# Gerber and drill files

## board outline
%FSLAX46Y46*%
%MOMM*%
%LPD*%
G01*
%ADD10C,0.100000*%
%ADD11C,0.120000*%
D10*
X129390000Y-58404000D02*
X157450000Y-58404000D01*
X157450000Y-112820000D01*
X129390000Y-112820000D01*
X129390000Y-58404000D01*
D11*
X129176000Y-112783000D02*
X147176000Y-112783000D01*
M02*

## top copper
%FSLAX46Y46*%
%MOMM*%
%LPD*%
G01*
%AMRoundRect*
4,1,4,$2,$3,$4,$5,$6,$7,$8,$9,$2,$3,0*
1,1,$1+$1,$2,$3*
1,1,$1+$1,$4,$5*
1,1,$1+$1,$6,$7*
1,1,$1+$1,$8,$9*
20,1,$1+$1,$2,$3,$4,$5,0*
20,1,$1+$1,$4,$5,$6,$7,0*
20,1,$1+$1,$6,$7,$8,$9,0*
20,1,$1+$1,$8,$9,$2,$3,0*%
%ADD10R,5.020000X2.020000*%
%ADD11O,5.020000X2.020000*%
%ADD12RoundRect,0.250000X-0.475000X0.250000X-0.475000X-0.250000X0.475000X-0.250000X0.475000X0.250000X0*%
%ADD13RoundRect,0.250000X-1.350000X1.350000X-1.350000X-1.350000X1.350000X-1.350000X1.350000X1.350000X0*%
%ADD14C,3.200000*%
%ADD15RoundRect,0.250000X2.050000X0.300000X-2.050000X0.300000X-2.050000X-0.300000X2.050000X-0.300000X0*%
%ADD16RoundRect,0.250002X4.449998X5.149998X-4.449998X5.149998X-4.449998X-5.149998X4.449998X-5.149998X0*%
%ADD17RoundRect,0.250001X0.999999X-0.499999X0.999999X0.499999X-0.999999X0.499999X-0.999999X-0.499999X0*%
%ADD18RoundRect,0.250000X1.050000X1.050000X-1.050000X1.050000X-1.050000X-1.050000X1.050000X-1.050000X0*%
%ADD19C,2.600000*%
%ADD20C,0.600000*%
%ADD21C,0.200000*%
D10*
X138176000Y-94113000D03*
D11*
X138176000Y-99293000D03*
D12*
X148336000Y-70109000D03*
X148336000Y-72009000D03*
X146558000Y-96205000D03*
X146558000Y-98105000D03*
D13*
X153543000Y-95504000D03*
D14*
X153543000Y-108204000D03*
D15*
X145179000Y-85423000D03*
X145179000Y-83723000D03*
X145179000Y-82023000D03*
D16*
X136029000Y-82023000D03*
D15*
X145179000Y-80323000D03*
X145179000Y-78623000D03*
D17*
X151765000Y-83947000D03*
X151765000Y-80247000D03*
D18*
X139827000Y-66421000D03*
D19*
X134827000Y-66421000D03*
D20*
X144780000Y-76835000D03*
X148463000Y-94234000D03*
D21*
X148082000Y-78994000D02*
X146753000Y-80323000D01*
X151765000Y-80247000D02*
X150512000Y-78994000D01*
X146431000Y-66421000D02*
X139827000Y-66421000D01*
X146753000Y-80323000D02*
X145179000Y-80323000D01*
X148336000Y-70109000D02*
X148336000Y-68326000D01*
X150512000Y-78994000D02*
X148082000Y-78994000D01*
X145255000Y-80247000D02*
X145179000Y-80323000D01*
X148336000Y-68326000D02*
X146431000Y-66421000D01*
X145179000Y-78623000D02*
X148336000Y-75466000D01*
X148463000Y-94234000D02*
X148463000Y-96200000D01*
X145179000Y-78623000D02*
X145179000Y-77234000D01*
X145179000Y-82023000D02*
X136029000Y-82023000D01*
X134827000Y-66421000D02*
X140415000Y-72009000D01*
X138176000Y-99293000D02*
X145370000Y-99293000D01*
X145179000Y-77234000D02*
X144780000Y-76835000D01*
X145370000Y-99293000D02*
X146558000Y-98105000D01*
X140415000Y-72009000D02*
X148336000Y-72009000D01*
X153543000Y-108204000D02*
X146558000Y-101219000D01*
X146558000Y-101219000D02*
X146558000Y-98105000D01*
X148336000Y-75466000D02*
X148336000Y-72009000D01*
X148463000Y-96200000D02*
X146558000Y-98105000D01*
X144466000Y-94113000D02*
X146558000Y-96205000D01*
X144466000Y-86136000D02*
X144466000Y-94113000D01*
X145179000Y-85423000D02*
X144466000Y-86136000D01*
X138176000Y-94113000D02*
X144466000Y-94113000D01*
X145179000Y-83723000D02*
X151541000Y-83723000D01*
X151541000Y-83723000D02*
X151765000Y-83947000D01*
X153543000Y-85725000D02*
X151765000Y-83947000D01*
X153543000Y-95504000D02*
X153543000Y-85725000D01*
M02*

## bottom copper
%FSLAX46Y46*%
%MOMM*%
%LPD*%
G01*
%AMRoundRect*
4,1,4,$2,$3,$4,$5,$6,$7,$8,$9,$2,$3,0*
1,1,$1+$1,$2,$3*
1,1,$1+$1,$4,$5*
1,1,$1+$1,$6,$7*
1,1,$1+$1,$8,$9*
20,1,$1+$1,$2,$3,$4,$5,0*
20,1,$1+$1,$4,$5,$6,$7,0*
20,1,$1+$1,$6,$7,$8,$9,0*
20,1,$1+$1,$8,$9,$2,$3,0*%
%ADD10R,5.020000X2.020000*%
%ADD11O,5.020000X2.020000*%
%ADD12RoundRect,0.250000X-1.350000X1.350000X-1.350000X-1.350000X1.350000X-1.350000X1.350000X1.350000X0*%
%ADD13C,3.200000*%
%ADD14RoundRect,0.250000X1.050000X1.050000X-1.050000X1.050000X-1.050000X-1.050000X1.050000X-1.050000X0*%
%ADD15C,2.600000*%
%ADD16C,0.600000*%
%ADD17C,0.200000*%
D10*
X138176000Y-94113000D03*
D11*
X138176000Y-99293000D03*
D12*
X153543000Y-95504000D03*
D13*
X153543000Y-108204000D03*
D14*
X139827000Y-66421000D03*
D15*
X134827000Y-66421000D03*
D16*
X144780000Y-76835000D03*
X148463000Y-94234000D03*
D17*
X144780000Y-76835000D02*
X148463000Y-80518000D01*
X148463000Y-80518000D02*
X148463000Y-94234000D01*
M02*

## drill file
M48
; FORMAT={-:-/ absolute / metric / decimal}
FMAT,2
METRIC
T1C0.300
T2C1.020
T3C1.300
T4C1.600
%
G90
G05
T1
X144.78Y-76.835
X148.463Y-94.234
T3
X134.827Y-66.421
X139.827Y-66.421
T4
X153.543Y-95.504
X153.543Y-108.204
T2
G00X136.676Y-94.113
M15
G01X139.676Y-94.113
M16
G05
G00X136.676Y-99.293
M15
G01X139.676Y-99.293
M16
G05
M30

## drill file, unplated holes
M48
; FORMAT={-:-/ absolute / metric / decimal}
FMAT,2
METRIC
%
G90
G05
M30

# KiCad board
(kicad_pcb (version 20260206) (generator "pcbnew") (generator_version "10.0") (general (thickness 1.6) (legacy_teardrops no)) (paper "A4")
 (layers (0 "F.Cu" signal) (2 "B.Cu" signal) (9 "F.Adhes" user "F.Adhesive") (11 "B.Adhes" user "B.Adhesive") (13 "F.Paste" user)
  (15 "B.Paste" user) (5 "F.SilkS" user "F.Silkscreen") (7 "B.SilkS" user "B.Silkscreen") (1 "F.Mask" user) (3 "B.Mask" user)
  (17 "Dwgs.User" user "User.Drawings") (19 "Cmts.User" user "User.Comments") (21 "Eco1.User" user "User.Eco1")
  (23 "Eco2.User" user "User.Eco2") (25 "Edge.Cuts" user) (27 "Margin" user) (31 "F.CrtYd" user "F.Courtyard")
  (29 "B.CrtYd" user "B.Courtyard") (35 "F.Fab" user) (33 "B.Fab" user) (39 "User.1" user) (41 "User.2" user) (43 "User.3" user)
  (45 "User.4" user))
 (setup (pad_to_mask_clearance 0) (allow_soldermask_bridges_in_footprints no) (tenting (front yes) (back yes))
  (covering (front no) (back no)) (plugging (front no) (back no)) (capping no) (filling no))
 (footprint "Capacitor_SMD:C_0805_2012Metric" (layer "F.Cu") (at 148.336 71.059 -90)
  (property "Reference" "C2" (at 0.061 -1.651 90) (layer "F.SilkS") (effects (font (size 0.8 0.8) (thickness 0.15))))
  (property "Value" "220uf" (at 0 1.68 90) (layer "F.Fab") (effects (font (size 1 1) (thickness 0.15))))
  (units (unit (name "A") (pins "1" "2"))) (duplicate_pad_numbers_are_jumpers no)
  (pad "1" smd roundrect (at -0.95 0 270) (size 1 1.45) (layers "F.Cu" "F.Mask" "F.Paste") (roundrect_rratio 0.25) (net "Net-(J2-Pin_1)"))
  (pad "2" smd roundrect (at 0.95 0 270) (size 1 1.45) (layers "F.Cu" "F.Mask" "F.Paste") (roundrect_rratio 0.25) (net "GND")))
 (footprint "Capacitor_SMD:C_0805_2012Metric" (layer "F.Cu") (at 146.558 97.155 -90)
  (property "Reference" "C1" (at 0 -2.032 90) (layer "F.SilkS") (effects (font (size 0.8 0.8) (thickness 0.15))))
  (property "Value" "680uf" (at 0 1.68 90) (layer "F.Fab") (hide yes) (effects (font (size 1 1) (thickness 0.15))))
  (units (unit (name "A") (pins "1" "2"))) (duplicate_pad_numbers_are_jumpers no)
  (pad "1" smd roundrect (at -0.95 0 270) (size 1 1.45) (layers "F.Cu" "F.Mask" "F.Paste") (roundrect_rratio 0.25) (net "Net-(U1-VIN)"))
  (pad "2" smd roundrect (at 0.95 0 270) (size 1 1.45) (layers "F.Cu" "F.Mask" "F.Paste") (roundrect_rratio 0.25) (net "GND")))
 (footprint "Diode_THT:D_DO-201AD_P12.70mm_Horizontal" (layer "F.Cu") (at 153.543 95.504 -90)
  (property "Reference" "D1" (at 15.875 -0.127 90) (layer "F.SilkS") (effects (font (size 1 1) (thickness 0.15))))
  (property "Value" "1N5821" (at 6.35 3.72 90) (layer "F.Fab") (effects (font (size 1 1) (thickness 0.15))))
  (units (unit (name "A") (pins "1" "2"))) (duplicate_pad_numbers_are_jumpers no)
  (pad "1" thru_hole roundrect (at 0 0 270) (size 3.2 3.2) (drill 1.6) (layers "*.Cu" "*.Mask") (remove_unused_layers no)
   (roundrect_rratio 0.078125) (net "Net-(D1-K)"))
  (pad "2" thru_hole circle (at 12.7 0 270) (size 3.2 3.2) (drill 1.6) (layers "*.Cu" "*.Mask") (remove_unused_layers no) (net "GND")))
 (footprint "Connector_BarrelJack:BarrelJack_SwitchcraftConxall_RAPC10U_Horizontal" (layer "F.Cu") (at 138.176 94.113 90)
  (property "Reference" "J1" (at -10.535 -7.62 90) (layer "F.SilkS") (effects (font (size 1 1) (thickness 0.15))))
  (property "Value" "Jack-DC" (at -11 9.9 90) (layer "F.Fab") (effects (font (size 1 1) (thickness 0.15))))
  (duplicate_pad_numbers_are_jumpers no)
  (fp_line (start -18.67 -9) (end -18.67 9) (stroke (width 0.12) (type solid)) (layer "Edge.Cuts"))
  (pad "1" thru_hole rect (at 0 0 90) (size 2.02 5.02) (drill oval 1.02 4.02) (layers "*.Cu" "*.Mask") (remove_unused_layers no)
   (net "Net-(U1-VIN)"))
  (pad "2" thru_hole oval (at -5.18 0 90) (size 2.02 5.02) (drill oval 1.02 4.02) (layers "*.Cu" "*.Mask") (remove_unused_layers no)
   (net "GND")))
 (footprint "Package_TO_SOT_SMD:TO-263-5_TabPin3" (layer "F.Cu") (at 137.529 82.023 180)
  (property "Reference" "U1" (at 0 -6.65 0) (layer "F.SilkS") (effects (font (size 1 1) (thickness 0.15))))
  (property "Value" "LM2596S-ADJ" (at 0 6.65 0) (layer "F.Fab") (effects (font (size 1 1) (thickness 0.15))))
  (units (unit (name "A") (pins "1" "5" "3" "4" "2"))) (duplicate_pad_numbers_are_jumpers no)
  (pad "" smd roundrect (at -0.925 -2.775 180) (size 4.55 5.25) (layers "F.Paste") (roundrect_rratio 0.054945))
  (pad "" smd roundrect (at -0.925 2.775 180) (size 4.55 5.25) (layers "F.Paste") (roundrect_rratio 0.054945))
  (pad "" smd roundrect (at 3.925 -2.775 180) (size 4.55 5.25) (layers "F.Paste") (roundrect_rratio 0.054945))
  (pad "" smd roundrect (at 3.925 2.775 180) (size 4.55 5.25) (layers "F.Paste") (roundrect_rratio 0.054945))
  (pad "1" smd roundrect (at -7.65 -3.4 180) (size 4.6 1.1) (layers "F.Cu" "F.Mask" "F.Paste") (roundrect_rratio 0.227273)
   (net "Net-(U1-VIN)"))
  (pad "2" smd roundrect (at -7.65 -1.7 180) (size 4.6 1.1) (layers "F.Cu" "F.Mask" "F.Paste") (roundrect_rratio 0.227273)
   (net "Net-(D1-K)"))
  (pad "3" smd roundrect (at -7.65 0 180) (size 4.6 1.1) (layers "F.Cu" "F.Mask" "F.Paste") (roundrect_rratio 0.227273) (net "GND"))
  (pad "3" smd roundrect (at 1.5 0 180) (size 9.4 10.8) (layers "F.Cu" "F.Mask") (roundrect_rratio 0.026596) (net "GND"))
  (pad "4" smd roundrect (at -7.65 1.7 180) (size 4.6 1.1) (layers "F.Cu" "F.Mask" "F.Paste") (roundrect_rratio 0.227273)
   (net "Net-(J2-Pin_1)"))
  (pad "5" smd roundrect (at -7.65 3.4 180) (size 4.6 1.1) (layers "F.Cu" "F.Mask" "F.Paste") (roundrect_rratio 0.227273) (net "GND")))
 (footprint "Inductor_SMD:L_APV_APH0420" (layer "F.Cu") (at 151.765 82.097 90)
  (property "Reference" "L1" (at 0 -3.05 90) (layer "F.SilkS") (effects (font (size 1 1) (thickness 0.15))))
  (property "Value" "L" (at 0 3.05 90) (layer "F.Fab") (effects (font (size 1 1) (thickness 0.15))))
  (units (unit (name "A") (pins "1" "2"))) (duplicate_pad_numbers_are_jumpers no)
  (pad "1" smd roundrect (at -1.85 0 90) (size 1.5 2.5) (layers "F.Cu" "F.Mask" "F.Paste") (roundrect_rratio 0.166667) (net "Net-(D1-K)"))
  (pad "2" smd roundrect (at 1.85 0 90) (size 1.5 2.5) (layers "F.Cu" "F.Mask" "F.Paste") (roundrect_rratio 0.166667) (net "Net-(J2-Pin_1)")))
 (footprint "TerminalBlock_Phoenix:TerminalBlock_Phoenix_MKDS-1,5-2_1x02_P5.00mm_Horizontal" (layer "F.Cu") (at 139.827 66.421 180)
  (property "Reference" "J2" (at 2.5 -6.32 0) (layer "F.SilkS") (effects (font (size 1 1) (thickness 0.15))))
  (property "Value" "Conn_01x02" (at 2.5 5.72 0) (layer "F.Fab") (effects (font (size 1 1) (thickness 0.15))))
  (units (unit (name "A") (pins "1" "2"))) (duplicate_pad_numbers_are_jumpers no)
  (pad "1" thru_hole roundrect (at 0 0 180) (size 2.6 2.6) (drill 1.3) (layers "*.Cu" "*.Mask") (remove_unused_layers no)
   (roundrect_rratio 0.096154) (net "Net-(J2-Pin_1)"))
  (pad "2" thru_hole circle (at 5 0 180) (size 2.6 2.6) (drill 1.3) (layers "*.Cu" "*.Mask") (remove_unused_layers no) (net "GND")))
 (gr_rect (start 129.39 58.404) (end 157.45 112.82) (stroke (width 0.1) (type solid)) (fill no) (layer "Edge.Cuts"))
 (segment (start 148.082 78.994) (end 146.753 80.323) (width 0.2) (layer "F.Cu") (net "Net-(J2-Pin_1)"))
 (segment (start 151.765 80.247) (end 150.512 78.994) (width 0.2) (layer "F.Cu") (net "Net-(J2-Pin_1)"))
 (segment (start 146.431 66.421) (end 139.827 66.421) (width 0.2) (layer "F.Cu") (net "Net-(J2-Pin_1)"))
 (segment (start 146.753 80.323) (end 145.179 80.323) (width 0.2) (layer "F.Cu") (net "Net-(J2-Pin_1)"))
 (segment (start 148.336 70.109) (end 148.336 68.326) (width 0.2) (layer "F.Cu") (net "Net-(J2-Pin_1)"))
 (segment (start 150.512 78.994) (end 148.082 78.994) (width 0.2) (layer "F.Cu") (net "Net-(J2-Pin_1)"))
 (segment (start 145.255 80.247) (end 145.179 80.323) (width 0.2) (layer "F.Cu") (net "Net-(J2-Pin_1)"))
 (segment (start 148.336 68.326) (end 146.431 66.421) (width 0.2) (layer "F.Cu") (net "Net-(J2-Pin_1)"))
 (segment (start 145.179 78.623) (end 148.336 75.466) (width 0.2) (layer "F.Cu") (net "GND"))
 (segment (start 148.463 94.234) (end 148.463 96.2) (width 0.2) (layer "F.Cu") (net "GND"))
 (segment (start 145.179 78.623) (end 145.179 77.234) (width 0.2) (layer "F.Cu") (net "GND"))
 (segment (start 145.179 82.023) (end 136.029 82.023) (width 0.2) (layer "F.Cu") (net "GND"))
 (segment (start 134.827 66.421) (end 140.415 72.009) (width 0.2) (layer "F.Cu") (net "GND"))
 (segment (start 138.176 99.293) (end 145.37 99.293) (width 0.2) (layer "F.Cu") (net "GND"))
 (segment (start 145.179 77.234) (end 144.78 76.835) (width 0.2) (layer "F.Cu") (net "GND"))
 (segment (start 145.37 99.293) (end 146.558 98.105) (width 0.2) (layer "F.Cu") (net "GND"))
 (segment (start 140.415 72.009) (end 148.336 72.009) (width 0.2) (layer "F.Cu") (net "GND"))
 (segment (start 153.543 108.204) (end 146.558 101.219) (width 0.2) (layer "F.Cu") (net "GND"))
 (segment (start 146.558 101.219) (end 146.558 98.105) (width 0.2) (layer "F.Cu") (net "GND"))
 (segment (start 148.336 75.466) (end 148.336 72.009) (width 0.2) (layer "F.Cu") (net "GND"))
 (segment (start 148.463 96.2) (end 146.558 98.105) (width 0.2) (layer "F.Cu") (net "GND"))
 (via (at 144.78 76.835) (size 0.6) (drill 0.3) (layers "F.Cu" "B.Cu") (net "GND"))
 (via (at 148.463 94.234) (size 0.6) (drill 0.3) (layers "F.Cu" "B.Cu") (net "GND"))
 (segment (start 144.78 76.835) (end 148.463 80.518) (width 0.2) (layer "B.Cu") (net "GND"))
 (segment (start 148.463 80.518) (end 148.463 94.234) (width 0.2) (layer "B.Cu") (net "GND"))
 (segment (start 144.466 94.113) (end 146.558 96.205) (width 0.2) (layer "F.Cu") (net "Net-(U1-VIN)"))
 (segment (start 144.466 86.136) (end 144.466 94.113) (width 0.2) (layer "F.Cu") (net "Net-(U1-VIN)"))
 (segment (start 145.179 85.423) (end 144.466 86.136) (width 0.2) (layer "F.Cu") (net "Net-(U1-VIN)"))
 (segment (start 138.176 94.113) (end 144.466 94.113) (width 0.2) (layer "F.Cu") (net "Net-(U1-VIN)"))
 (segment (start 145.179 83.723) (end 151.541 83.723) (width 0.2) (layer "F.Cu") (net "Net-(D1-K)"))
 (segment (start 151.541 83.723) (end 151.765 83.947) (width 0.2) (layer "F.Cu") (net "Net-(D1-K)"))
 (segment (start 153.543 85.725) (end 151.765 83.947) (width 0.2) (layer "F.Cu") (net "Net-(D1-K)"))
 (segment (start 153.543 95.504) (end 153.543 85.725) (width 0.2) (layer "F.Cu") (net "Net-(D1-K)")))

